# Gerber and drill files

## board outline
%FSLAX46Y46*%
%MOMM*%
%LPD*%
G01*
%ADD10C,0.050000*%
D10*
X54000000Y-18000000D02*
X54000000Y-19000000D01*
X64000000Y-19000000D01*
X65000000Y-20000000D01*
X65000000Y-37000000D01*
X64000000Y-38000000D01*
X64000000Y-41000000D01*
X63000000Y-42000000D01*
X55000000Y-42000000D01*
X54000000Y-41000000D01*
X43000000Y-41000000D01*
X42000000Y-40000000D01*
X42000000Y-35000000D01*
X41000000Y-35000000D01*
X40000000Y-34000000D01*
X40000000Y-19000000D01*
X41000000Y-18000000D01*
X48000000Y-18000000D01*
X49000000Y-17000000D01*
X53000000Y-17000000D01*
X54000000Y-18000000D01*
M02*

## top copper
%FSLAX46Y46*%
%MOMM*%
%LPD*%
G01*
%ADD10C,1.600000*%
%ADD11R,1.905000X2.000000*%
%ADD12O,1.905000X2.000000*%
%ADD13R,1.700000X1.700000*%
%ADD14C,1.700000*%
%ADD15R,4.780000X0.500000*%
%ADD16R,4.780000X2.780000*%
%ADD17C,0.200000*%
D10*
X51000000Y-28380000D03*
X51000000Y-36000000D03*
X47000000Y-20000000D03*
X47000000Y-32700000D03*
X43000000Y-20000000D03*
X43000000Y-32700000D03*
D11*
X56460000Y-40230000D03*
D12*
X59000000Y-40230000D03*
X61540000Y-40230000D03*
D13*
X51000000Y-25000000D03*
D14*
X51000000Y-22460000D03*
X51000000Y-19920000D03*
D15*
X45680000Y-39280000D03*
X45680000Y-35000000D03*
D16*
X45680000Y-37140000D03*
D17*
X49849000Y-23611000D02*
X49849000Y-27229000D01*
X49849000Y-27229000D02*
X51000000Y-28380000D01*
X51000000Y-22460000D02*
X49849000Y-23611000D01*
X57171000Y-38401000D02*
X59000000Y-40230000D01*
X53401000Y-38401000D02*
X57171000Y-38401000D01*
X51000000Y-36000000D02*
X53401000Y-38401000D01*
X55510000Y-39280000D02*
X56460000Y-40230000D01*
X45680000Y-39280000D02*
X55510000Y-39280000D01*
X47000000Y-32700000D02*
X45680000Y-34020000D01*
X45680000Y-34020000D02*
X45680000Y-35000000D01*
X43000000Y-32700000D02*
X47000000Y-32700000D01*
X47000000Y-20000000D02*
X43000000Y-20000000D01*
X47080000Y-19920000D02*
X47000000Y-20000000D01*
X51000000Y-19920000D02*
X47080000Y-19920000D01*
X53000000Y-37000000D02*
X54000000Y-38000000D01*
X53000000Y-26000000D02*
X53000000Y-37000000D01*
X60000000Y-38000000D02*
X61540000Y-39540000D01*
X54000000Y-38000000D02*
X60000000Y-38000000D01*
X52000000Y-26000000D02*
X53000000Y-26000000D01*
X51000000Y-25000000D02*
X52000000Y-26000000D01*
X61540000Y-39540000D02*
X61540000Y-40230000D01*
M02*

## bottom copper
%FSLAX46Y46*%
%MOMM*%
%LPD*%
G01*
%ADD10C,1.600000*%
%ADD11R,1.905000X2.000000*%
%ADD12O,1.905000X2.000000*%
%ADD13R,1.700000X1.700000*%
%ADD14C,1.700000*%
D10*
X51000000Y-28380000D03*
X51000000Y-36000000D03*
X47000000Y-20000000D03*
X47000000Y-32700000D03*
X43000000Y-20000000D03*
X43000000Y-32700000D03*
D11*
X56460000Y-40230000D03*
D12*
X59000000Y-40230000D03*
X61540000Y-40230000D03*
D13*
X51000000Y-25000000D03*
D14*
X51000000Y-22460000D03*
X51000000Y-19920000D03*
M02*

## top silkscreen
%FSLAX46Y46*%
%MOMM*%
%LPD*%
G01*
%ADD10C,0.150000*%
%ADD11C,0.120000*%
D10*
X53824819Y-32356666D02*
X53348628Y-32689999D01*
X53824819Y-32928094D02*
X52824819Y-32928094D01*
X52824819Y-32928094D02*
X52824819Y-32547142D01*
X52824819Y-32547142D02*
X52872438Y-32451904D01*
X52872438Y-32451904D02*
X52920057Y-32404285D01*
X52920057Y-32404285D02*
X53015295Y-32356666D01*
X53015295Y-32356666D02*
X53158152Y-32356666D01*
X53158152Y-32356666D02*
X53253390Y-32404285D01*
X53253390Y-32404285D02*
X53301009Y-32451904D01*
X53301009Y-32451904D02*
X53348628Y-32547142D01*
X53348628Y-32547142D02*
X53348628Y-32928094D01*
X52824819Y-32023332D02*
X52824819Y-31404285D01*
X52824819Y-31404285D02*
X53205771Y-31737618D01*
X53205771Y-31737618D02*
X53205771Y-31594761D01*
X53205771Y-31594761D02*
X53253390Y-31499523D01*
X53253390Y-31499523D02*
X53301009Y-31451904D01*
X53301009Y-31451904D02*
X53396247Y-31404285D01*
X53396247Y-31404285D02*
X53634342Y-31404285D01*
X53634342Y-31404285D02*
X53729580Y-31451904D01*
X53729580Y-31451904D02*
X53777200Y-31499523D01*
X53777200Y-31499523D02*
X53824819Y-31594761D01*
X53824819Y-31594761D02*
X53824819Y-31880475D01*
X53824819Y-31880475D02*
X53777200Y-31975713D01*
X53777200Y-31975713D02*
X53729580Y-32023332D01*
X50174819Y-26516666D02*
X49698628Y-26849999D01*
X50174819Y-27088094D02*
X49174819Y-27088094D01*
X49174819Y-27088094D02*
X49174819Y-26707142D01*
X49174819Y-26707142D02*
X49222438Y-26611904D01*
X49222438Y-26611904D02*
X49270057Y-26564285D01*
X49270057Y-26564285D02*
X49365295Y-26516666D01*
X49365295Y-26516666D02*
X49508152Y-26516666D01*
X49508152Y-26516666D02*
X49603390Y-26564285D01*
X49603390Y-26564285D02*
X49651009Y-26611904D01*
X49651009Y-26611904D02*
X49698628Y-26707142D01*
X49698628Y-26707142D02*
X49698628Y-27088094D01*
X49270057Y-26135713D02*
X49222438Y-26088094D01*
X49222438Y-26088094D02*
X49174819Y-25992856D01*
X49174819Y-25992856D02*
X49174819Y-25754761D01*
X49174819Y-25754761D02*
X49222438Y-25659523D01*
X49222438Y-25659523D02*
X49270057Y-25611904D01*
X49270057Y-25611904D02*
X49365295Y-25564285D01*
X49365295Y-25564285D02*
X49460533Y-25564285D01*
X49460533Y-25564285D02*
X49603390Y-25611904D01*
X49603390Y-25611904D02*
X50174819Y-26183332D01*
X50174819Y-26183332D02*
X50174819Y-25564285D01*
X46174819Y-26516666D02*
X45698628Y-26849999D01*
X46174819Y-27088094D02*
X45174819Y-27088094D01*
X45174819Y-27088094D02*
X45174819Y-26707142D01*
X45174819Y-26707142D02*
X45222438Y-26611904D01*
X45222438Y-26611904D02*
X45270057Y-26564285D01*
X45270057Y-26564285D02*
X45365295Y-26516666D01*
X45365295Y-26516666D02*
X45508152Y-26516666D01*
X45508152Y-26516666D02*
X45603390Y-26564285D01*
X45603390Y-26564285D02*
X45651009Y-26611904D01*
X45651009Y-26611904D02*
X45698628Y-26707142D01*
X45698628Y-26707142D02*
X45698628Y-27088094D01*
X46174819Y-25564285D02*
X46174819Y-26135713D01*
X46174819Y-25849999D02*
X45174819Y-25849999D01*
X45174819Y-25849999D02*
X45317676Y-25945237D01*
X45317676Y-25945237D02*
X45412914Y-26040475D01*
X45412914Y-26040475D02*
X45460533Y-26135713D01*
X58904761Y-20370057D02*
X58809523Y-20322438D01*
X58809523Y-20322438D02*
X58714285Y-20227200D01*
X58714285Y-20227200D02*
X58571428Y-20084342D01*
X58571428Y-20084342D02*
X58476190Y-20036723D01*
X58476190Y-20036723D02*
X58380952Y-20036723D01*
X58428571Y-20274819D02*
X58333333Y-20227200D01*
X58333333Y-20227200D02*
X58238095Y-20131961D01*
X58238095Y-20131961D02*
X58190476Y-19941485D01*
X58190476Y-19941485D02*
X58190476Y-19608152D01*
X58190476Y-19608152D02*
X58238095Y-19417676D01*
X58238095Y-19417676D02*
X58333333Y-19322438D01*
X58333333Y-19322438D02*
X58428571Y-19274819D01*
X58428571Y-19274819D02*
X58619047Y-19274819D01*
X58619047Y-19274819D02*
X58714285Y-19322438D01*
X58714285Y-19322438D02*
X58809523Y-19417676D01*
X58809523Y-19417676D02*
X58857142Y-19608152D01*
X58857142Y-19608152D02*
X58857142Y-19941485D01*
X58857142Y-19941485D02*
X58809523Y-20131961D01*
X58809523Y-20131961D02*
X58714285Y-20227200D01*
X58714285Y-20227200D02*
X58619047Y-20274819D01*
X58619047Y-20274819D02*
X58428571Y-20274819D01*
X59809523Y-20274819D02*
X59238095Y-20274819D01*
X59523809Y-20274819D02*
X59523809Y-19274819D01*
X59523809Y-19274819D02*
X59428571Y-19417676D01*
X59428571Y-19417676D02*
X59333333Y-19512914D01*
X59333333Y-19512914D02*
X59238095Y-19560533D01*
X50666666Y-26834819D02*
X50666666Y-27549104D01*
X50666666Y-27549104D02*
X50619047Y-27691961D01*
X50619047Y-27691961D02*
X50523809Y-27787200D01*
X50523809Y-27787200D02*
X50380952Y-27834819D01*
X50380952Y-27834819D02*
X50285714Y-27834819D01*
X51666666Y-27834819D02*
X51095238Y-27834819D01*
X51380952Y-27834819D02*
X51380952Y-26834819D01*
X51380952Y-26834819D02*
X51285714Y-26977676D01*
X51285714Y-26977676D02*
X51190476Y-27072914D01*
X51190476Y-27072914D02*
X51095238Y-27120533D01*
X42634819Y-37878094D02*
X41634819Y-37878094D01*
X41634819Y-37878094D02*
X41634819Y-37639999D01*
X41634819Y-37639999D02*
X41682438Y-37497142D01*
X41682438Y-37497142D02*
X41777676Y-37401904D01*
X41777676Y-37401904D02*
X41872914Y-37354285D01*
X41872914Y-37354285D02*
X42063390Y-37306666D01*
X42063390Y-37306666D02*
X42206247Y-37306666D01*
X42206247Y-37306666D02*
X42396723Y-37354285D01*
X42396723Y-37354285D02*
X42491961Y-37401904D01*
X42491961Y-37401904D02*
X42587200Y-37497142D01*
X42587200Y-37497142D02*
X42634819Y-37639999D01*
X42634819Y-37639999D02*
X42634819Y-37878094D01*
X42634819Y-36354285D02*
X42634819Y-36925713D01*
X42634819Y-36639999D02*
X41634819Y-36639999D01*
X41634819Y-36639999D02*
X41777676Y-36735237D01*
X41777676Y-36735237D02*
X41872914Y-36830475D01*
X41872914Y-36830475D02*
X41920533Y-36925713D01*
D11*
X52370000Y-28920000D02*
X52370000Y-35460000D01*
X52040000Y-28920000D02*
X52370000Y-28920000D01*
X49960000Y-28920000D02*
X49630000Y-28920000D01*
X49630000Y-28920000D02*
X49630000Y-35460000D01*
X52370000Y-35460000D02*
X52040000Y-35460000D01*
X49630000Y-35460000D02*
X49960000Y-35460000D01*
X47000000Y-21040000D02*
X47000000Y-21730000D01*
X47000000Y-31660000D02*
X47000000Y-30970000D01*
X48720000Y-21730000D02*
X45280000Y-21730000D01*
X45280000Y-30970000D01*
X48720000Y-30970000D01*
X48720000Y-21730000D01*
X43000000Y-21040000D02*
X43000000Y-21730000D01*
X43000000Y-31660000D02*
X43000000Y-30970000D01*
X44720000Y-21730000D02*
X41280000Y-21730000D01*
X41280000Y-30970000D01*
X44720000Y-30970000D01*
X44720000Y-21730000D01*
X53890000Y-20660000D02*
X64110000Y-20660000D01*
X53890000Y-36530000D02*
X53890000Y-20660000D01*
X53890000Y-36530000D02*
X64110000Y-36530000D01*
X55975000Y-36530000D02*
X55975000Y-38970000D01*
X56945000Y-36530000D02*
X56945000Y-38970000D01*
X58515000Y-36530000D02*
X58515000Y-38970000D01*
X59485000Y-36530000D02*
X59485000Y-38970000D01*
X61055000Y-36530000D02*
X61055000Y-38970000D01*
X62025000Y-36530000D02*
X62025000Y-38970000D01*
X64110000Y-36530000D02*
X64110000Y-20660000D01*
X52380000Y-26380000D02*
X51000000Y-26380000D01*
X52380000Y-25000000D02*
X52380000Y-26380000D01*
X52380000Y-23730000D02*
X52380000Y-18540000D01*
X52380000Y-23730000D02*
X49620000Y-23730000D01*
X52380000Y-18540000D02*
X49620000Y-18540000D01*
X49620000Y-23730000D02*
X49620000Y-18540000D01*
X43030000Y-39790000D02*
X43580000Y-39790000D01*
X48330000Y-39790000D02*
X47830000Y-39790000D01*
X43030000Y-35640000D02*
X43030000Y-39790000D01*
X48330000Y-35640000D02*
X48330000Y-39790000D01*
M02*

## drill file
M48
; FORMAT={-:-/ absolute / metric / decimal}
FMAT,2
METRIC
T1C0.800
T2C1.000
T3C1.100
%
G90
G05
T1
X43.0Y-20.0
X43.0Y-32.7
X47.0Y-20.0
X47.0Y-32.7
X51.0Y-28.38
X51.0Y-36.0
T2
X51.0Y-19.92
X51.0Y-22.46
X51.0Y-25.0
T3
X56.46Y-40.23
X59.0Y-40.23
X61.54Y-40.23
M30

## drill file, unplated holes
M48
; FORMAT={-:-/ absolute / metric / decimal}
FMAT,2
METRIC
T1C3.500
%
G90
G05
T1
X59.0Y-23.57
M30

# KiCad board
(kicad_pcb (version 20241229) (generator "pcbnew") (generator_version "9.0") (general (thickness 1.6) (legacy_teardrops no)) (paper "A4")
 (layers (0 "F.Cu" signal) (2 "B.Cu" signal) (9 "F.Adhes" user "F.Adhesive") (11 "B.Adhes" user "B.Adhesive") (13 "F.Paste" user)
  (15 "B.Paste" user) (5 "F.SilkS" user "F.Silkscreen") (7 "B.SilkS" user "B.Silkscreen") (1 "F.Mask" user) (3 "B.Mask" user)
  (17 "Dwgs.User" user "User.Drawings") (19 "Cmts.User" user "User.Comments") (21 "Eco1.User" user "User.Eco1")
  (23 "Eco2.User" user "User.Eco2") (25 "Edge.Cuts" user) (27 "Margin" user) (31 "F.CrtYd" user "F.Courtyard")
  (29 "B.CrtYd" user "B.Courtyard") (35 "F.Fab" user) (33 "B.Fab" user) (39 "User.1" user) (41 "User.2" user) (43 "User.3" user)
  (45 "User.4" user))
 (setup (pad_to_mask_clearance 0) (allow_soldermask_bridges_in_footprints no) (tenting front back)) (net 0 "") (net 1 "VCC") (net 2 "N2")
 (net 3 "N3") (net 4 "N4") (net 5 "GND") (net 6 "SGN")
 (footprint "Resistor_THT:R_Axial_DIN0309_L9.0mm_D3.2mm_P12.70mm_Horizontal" (layer "F.Cu") (at 47 20 -90)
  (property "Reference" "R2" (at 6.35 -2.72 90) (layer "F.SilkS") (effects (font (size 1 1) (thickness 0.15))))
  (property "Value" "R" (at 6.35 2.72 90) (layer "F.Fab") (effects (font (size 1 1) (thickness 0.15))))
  (fp_line (start 1.04 0) (end 1.73 0) (stroke (width 0.12) (type solid)) (layer "F.SilkS"))
  (fp_line (start 11.66 0) (end 10.97 0) (stroke (width 0.12) (type solid)) (layer "F.SilkS"))
  (fp_rect (start 1.73 -1.72) (end 10.97 1.72) (stroke (width 0.12) (type solid)) (fill no) (layer "F.SilkS"))
  (pad "1" thru_hole circle (at 0 0 270) (size 1.6 1.6) (drill 0.8) (layers "*.Cu" "*.Mask") (remove_unused_layers no) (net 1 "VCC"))
  (pad "2" thru_hole circle (at 12.7 0 270) (size 1.6 1.6) (drill 0.8) (layers "*.Cu" "*.Mask") (remove_unused_layers no) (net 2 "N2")))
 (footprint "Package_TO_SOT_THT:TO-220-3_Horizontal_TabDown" (layer "F.Cu") (at 56.46 40.23)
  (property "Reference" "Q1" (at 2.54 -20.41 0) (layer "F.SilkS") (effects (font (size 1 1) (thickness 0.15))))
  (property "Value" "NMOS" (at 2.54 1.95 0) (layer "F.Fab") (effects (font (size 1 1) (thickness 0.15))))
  (fp_line (start -2.57 -19.57) (end 7.65 -19.57) (stroke (width 0.12) (type solid)) (layer "F.SilkS"))
  (fp_line (start -2.57 -3.7) (end -2.57 -19.57) (stroke (width 0.12) (type solid)) (layer "F.SilkS"))
  (fp_line (start -2.57 -3.7) (end 7.65 -3.7) (stroke (width 0.12) (type solid)) (layer "F.SilkS"))
  (fp_line (start -0.485 -3.7) (end -0.485 -1.26) (stroke (width 0.12) (type solid)) (layer "F.SilkS"))
  (fp_line (start 0.485 -3.7) (end 0.485 -1.26) (stroke (width 0.12) (type solid)) (layer "F.SilkS"))
  (fp_line (start 2.055 -3.7) (end 2.055 -1.26) (stroke (width 0.12) (type solid)) (layer "F.SilkS"))
  (fp_line (start 3.025 -3.7) (end 3.025 -1.26) (stroke (width 0.12) (type solid)) (layer "F.SilkS"))
  (fp_line (start 4.595 -3.7) (end 4.595 -1.26) (stroke (width 0.12) (type solid)) (layer "F.SilkS"))
  (fp_line (start 5.565 -3.7) (end 5.565 -1.26) (stroke (width 0.12) (type solid)) (layer "F.SilkS"))
  (fp_line (start 7.65 -3.7) (end 7.65 -19.57) (stroke (width 0.12) (type solid)) (layer "F.SilkS"))
  (pad "" np_thru_hole circle (at 2.54 -16.66) (size 3.5 3.5) (drill 3.5) (layers "*.Cu" "*.Mask"))
  (pad "1" thru_hole rect (at 0 0) (size 1.905 2) (drill 1.1) (layers "*.Cu" "*.Mask") (remove_unused_layers no) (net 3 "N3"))
  (pad "2" thru_hole oval (at 2.54 0) (size 1.905 2) (drill 1.1) (layers "*.Cu" "*.Mask") (remove_unused_layers no) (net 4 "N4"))
  (pad "3" thru_hole oval (at 5.08 0) (size 1.905 2) (drill 1.1) (layers "*.Cu" "*.Mask") (remove_unused_layers no) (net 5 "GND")))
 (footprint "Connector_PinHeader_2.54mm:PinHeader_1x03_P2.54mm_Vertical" (layer "F.Cu") (at 51 25 180)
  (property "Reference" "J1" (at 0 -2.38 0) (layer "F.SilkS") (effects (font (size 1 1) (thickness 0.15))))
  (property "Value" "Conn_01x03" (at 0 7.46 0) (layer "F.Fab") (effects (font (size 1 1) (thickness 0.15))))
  (fp_line (start 1.38 1.27) (end 1.38 6.46) (stroke (width 0.12) (type solid)) (layer "F.SilkS"))
  (fp_line (start -1.38 6.46) (end 1.38 6.46) (stroke (width 0.12) (type solid)) (layer "F.SilkS"))
  (fp_line (start -1.38 1.27) (end 1.38 1.27) (stroke (width 0.12) (type solid)) (layer "F.SilkS"))
  (fp_line (start -1.38 1.27) (end -1.38 6.46) (stroke (width 0.12) (type solid)) (layer "F.SilkS"))
  (fp_line (start -1.38 0) (end -1.38 -1.38) (stroke (width 0.12) (type solid)) (layer "F.SilkS"))
  (fp_line (start -1.38 -1.38) (end 0 -1.38) (stroke (width 0.12) (type solid)) (layer "F.SilkS"))
  (pad "1" thru_hole rect (at 0 0 180) (size 1.7 1.7) (drill 1) (layers "*.Cu" "*.Mask") (remove_unused_layers no) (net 5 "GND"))
  (pad "2" thru_hole circle (at 0 2.54 180) (size 1.7 1.7) (drill 1) (layers "*.Cu" "*.Mask") (remove_unused_layers no) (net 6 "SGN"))
  (pad "3" thru_hole circle (at 0 5.08 180) (size 1.7 1.7) (drill 1) (layers "*.Cu" "*.Mask") (remove_unused_layers no) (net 1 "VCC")))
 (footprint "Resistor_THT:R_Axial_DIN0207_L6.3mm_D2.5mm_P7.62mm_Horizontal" (layer "F.Cu") (at 51 28.38 -90)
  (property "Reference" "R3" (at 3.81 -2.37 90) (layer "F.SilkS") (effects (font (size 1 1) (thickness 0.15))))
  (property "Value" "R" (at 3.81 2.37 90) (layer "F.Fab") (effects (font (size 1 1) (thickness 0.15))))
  (fp_line (start 0.54 1.37) (end 7.08 1.37) (stroke (width 0.12) (type solid)) (layer "F.SilkS"))
  (fp_line (start 7.08 1.37) (end 7.08 1.04) (stroke (width 0.12) (type solid)) (layer "F.SilkS"))
  (fp_line (start 0.54 1.04) (end 0.54 1.37) (stroke (width 0.12) (type solid)) (layer "F.SilkS"))
  (fp_line (start 0.54 -1.04) (end 0.54 -1.37) (stroke (width 0.12) (type solid)) (layer "F.SilkS"))
  (fp_line (start 0.54 -1.37) (end 7.08 -1.37) (stroke (width 0.12) (type solid)) (layer "F.SilkS"))
  (fp_line (start 7.08 -1.37) (end 7.08 -1.04) (stroke (width 0.12) (type solid)) (layer "F.SilkS"))
  (pad "1" thru_hole circle (at 0 0 270) (size 1.6 1.6) (drill 0.8) (layers "*.Cu" "*.Mask") (remove_unused_layers no) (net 6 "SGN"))
  (pad "2" thru_hole circle (at 7.62 0 270) (size 1.6 1.6) (drill 0.8) (layers "*.Cu" "*.Mask") (remove_unused_layers no) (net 4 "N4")))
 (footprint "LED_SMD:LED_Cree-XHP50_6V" (layer "F.Cu") (at 45.68 37.14 90)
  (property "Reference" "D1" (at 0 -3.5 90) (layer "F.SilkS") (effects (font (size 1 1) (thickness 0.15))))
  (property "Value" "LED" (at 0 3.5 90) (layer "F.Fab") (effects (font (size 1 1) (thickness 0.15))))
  (fp_line (start 1.5 -2.65) (end -2.65 -2.65) (stroke (width 0.12) (type solid)) (layer "F.SilkS"))
  (fp_line (start -2.65 -2.65) (end -2.65 -2.1) (stroke (width 0.12) (type solid)) (layer "F.SilkS"))
  (fp_line (start 1.5 2.65) (end -2.65 2.65) (stroke (width 0.12) (type solid)) (layer "F.SilkS"))
  (fp_line (start -2.65 2.65) (end -2.65 2.15) (stroke (width 0.12) (type solid)) (layer "F.SilkS"))
  (pad "" smd rect (at -2.14 -1.32 90) (size 0.5 2.14) (layers "F.Paste"))
  (pad "" smd rect (at -2.14 1.32 90) (size 0.5 2.14) (layers "F.Paste"))
  (pad "" smd rect (at -0.61 -1.575 90) (size 0.97 0.8) (layers "F.Paste"))
  (pad "" smd rect (at -0.61 -0.525 90) (size 0.97 0.8) (layers "F.Paste"))
  (pad "" smd rect (at -0.61 0.525 90) (size 0.97 0.8) (layers "F.Paste"))
  (pad "" smd rect (at -0.61 1.575 90) (size 0.97 0.8) (layers "F.Paste"))
  (pad "" smd rect (at 0.61 -1.575 90) (size 0.97 0.8) (layers "F.Paste"))
  (pad "" smd rect (at 0.61 -0.525 90) (size 0.97 0.8) (layers "F.Paste"))
  (pad "" smd rect (at 0.61 0.525 90) (size 0.97 0.8) (layers "F.Paste"))
  (pad "" smd rect (at 0.61 1.575 90) (size 0.97 0.8) (layers "F.Paste"))
  (pad "" smd rect (at 2.14 -1.32 90) (size 0.5 2.14) (layers "F.Paste"))
  (pad "" smd rect (at 2.14 1.32 90) (size 0.5 2.14) (layers "F.Paste"))
  (pad "1" smd rect (at -2.14 0 90) (size 0.5 4.78) (layers "F.Cu" "F.Mask") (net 3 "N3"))
  (pad "2" smd rect (at 2.14 0 90) (size 0.5 4.78) (layers "F.Cu" "F.Mask") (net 2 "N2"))
  (pad "3" smd rect (at 0 0 90) (size 2.78 4.78) (layers "F.Cu" "F.Mask")))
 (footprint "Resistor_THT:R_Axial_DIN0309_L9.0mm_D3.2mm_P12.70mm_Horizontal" (layer "F.Cu") (at 43 20 -90)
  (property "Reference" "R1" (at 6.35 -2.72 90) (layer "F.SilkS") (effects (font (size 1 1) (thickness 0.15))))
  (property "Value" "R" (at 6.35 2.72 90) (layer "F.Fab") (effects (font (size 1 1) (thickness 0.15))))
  (fp_line (start 1.04 0) (end 1.73 0) (stroke (width 0.12) (type solid)) (layer "F.SilkS"))
  (fp_line (start 11.66 0) (end 10.97 0) (stroke (width 0.12) (type solid)) (layer "F.SilkS"))
  (fp_rect (start 1.73 -1.72) (end 10.97 1.72) (stroke (width 0.12) (type solid)) (fill no) (layer "F.SilkS"))
  (pad "1" thru_hole circle (at 0 0 270) (size 1.6 1.6) (drill 0.8) (layers "*.Cu" "*.Mask") (remove_unused_layers no) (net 1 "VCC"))
  (pad "2" thru_hole circle (at 12.7 0 270) (size 1.6 1.6) (drill 0.8) (layers "*.Cu" "*.Mask") (remove_unused_layers no) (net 2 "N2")))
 (gr_poly
  (pts (xy 41 18) (xy 40 19) (xy 40 34) (xy 41 35) (xy 42 35) (xy 42 40) (xy 43 41) (xy 54 41) (xy 55 42) (xy 63 42) (xy 64 41) (xy 64 38)
   (xy 65 37) (xy 65 20) (xy 64 19) (xy 54 19) (xy 54 18) (xy 53 17) (xy 49 17) (xy 48 18))
  (stroke (width 0.05) (type solid)) (fill no) (layer "Edge.Cuts"))
 (segment (start 45.68 39.28) (end 55.51 39.28) (width 0.2) (layer "F.Cu") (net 3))
 (segment (start 55.51 39.28) (end 56.46 40.23) (width 0.2) (layer "F.Cu") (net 3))
 (segment (start 47 32.7) (end 45.68 34.02) (width 0.2) (layer "F.Cu") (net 2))
 (segment (start 43 32.7) (end 47 32.7) (width 0.2) (layer "F.Cu") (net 2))
 (segment (start 45.68 34.02) (end 45.68 35) (width 0.2) (layer "F.Cu") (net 2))
 (segment (start 49.849 23.611) (end 49.849 27.229) (width 0.2) (layer "F.Cu") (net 6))
 (segment (start 49.849 27.229) (end 51 28.38) (width 0.2) (layer "F.Cu") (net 6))
 (segment (start 51 22.46) (end 49.849 23.611) (width 0.2) (layer "F.Cu") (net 6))
 (segment (start 47 20) (end 43 20) (width 0.2) (layer "F.Cu") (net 1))
 (segment (start 47.08 19.92) (end 47 20) (width 0.2) (layer "F.Cu") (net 1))
 (segment (start 51 19.92) (end 47.08 19.92) (width 0.2) (layer "F.Cu") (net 1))
 (segment (start 53 26) (end 53 37) (width 0.2) (layer "F.Cu") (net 5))
 (segment (start 60 38) (end 61.54 39.54) (width 0.2) (layer "F.Cu") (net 5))
 (segment (start 51 25) (end 52 26) (width 0.2) (layer "F.Cu") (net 5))
 (segment (start 61.54 39.54) (end 61.54 40.23) (width 0.2) (layer "F.Cu") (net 5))
 (segment (start 53 37) (end 54 38) (width 0.2) (layer "F.Cu") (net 5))
 (segment (start 54 38) (end 60 38) (width 0.2) (layer "F.Cu") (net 5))
 (segment (start 52 26) (end 53 26) (width 0.2) (layer "F.Cu") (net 5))
 (segment (start 51 36) (end 53.401 38.401) (width 0.2) (layer "F.Cu") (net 4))
 (segment (start 57.171 38.401) (end 59 40.23) (width 0.2) (layer "F.Cu") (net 4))
 (segment (start 53.401 38.401) (end 57.171 38.401) (width 0.2) (layer "F.Cu") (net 4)))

